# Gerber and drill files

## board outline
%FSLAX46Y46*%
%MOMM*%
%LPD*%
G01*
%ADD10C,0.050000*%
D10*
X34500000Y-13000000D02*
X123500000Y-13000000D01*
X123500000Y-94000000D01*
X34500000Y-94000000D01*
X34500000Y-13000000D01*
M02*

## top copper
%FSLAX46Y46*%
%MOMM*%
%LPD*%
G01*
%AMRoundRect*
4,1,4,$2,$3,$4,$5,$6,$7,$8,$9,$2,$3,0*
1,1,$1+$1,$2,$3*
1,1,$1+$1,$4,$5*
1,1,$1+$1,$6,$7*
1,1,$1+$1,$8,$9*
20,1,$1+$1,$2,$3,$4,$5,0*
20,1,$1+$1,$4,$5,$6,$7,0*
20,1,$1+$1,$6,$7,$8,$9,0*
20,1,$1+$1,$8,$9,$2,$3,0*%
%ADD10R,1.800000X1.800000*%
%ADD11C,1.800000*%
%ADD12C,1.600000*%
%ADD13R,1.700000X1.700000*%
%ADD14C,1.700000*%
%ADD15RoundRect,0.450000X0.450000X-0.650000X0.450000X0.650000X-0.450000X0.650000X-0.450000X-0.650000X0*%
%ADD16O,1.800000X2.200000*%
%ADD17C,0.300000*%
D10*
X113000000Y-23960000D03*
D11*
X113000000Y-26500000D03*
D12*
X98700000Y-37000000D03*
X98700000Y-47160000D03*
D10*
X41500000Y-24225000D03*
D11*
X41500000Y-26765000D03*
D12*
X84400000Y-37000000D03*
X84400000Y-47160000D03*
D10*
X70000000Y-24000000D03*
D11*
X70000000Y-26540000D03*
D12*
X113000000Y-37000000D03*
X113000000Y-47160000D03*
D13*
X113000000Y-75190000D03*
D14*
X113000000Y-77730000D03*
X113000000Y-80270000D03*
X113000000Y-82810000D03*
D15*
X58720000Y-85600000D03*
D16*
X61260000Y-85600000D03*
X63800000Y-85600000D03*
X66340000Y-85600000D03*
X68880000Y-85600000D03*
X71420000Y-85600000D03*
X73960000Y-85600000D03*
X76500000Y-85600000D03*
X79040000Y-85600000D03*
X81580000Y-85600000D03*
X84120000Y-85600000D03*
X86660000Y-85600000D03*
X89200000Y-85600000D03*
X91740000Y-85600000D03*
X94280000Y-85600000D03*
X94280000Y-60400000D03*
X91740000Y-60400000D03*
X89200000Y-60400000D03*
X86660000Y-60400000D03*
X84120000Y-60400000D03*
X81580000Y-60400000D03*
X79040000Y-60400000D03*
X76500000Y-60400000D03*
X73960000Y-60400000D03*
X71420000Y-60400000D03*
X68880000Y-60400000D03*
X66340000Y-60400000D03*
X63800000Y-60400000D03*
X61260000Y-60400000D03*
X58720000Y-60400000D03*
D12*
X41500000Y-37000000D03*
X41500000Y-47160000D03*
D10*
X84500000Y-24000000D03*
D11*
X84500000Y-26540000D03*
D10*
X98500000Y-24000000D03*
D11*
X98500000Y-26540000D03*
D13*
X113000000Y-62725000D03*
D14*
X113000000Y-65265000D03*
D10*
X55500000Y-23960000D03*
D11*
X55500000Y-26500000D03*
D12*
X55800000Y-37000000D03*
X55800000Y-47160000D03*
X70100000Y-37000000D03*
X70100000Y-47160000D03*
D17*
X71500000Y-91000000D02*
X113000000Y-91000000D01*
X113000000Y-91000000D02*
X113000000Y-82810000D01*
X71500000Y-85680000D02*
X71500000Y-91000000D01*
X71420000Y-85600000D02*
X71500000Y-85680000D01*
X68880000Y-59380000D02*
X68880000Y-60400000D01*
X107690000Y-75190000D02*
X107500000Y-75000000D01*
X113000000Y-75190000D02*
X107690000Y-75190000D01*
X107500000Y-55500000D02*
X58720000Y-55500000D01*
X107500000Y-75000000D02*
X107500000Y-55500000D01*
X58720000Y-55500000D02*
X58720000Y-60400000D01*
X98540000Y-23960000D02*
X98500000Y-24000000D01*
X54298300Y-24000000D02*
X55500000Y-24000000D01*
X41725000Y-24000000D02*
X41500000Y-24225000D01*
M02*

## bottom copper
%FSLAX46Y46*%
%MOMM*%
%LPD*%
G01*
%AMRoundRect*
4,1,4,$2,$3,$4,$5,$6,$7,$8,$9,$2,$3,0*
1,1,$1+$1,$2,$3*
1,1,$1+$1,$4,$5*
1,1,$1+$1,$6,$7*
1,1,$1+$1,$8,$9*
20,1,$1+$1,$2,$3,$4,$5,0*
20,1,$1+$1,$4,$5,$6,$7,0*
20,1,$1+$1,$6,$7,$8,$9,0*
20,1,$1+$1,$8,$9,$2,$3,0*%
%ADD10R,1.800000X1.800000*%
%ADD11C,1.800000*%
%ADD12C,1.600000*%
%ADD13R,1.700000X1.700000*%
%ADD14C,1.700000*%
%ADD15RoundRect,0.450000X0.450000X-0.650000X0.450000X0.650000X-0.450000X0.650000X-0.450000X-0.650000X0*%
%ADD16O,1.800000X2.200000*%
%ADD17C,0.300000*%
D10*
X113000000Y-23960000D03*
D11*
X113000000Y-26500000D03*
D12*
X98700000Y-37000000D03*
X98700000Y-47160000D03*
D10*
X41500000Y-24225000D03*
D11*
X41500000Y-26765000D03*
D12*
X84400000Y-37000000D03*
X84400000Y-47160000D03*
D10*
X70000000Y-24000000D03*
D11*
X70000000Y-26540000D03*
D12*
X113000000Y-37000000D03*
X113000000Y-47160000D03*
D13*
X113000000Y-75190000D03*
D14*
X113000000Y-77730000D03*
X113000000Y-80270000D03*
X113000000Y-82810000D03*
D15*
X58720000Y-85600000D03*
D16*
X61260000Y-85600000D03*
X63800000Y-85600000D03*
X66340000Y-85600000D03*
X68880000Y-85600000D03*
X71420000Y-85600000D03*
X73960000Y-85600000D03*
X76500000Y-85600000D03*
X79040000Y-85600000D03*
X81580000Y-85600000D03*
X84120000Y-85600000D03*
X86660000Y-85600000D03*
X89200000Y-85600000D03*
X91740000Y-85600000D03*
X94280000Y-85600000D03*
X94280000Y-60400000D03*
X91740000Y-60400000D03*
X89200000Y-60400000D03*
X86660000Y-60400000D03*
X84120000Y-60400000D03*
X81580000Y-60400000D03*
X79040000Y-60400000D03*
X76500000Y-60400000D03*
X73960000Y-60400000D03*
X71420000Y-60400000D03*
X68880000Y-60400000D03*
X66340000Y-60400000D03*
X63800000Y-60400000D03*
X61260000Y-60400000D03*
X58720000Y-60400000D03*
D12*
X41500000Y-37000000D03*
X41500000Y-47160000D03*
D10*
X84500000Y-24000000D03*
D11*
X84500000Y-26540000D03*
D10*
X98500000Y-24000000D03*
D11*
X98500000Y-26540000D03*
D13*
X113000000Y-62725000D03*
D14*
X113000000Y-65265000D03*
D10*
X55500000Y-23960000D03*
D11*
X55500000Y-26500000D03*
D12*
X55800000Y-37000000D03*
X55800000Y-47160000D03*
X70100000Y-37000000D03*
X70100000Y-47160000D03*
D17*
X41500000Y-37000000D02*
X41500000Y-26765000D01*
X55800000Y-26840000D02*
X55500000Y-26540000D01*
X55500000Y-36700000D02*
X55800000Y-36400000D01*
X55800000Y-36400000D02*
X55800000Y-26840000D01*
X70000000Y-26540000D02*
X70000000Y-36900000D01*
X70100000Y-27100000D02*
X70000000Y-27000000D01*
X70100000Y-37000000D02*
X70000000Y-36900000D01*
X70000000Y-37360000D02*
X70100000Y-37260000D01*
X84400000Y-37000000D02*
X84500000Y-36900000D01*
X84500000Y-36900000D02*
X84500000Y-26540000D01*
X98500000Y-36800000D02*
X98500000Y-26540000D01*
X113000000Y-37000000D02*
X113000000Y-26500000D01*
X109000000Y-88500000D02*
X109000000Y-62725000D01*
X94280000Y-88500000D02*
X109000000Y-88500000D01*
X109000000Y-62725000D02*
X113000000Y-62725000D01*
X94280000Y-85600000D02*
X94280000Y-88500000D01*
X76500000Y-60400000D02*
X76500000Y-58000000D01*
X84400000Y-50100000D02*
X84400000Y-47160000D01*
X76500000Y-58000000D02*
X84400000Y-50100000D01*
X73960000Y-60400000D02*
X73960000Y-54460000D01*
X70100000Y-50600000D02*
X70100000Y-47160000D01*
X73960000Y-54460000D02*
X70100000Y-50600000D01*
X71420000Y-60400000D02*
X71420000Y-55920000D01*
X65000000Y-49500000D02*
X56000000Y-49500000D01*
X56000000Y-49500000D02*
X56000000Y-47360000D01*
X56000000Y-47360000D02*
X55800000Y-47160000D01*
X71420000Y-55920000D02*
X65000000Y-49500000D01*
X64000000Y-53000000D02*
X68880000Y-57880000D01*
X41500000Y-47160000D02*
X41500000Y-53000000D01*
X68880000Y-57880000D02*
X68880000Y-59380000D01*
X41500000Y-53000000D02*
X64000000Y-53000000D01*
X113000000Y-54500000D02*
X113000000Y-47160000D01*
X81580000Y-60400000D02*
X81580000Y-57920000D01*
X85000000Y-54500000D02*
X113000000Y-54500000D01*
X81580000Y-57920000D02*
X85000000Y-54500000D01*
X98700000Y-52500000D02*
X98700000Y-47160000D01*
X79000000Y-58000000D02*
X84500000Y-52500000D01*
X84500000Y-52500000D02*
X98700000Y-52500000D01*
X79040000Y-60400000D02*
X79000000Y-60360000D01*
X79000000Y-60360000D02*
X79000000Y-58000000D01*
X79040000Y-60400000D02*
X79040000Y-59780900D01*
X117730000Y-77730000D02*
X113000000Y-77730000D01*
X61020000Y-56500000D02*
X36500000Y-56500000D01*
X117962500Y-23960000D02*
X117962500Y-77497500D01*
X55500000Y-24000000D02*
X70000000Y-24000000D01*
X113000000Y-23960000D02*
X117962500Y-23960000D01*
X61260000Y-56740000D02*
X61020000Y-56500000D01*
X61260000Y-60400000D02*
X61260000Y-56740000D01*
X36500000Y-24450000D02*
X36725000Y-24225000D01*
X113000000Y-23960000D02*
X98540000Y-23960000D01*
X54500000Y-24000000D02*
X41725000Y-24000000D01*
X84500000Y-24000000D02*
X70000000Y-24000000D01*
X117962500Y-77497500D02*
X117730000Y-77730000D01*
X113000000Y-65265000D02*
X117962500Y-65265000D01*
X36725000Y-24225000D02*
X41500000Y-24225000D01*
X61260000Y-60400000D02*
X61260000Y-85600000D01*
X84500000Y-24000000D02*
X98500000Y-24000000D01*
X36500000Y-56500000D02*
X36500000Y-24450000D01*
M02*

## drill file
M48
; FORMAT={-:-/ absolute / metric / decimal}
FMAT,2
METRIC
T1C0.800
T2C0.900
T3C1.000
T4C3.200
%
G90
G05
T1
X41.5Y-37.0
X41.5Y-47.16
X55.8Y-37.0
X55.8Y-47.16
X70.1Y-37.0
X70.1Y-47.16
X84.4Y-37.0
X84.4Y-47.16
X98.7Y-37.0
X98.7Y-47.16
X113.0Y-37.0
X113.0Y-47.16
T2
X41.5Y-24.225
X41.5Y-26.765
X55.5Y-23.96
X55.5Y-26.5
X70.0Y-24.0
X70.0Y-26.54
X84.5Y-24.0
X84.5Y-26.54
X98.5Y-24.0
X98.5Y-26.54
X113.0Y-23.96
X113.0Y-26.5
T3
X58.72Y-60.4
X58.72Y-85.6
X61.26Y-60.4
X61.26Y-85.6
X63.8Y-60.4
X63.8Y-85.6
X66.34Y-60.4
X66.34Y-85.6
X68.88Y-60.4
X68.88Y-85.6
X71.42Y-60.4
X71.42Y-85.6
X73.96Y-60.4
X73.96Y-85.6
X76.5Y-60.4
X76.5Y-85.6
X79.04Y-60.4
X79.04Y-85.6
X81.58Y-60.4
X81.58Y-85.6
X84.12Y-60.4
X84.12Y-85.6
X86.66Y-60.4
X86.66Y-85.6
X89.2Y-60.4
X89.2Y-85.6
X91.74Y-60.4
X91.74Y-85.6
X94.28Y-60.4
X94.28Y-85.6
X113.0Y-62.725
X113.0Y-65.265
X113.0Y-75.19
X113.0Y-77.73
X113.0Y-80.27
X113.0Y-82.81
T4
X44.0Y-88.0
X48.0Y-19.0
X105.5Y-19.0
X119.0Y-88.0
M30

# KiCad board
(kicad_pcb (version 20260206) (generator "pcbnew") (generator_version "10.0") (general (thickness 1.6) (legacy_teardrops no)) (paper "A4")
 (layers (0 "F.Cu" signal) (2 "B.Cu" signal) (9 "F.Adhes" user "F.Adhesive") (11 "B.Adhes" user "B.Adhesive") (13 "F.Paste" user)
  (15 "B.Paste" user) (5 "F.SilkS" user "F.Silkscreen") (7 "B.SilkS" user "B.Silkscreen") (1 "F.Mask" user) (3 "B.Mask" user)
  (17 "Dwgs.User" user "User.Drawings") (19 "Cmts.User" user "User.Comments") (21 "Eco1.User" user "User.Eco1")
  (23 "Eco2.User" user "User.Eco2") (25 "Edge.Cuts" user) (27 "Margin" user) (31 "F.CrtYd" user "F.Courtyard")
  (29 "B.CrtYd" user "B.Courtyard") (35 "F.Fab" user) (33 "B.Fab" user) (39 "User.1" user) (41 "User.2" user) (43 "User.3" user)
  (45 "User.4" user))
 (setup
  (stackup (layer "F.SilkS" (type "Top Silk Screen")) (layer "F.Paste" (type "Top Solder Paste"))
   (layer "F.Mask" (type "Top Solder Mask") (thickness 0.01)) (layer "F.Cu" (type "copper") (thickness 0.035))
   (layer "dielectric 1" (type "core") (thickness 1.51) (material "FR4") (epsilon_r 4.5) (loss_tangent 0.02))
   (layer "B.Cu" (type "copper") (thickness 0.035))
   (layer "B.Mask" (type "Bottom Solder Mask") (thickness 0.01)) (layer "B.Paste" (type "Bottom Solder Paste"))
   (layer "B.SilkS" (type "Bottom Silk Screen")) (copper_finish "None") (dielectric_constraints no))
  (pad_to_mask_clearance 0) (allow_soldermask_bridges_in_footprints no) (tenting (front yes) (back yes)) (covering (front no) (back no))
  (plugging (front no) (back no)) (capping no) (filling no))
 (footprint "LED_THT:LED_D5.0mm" (layer "F.Cu") (at 113 23.96 -90)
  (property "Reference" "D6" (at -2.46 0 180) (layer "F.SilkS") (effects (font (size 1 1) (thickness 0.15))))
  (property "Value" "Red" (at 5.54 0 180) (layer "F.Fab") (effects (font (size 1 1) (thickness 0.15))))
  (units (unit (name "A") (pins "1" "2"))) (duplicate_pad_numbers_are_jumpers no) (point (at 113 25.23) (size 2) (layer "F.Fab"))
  (pad "1" thru_hole rect (at 0 0 270) (size 1.8 1.8) (drill 0.9) (layers "*.Cu" "*.Mask") (remove_unused_layers no) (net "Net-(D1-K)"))
  (pad "2" thru_hole circle (at 2.54 0 270) (size 1.8 1.8) (drill 0.9) (layers "*.Cu" "*.Mask") (remove_unused_layers no) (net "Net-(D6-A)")))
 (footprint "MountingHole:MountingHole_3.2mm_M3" (layer "F.Cu") (at 44 88)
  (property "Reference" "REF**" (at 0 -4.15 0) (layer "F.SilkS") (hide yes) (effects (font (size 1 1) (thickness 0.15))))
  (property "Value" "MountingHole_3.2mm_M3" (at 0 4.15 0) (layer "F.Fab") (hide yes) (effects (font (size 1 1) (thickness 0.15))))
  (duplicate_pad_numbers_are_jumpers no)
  (pad "" np_thru_hole circle (at 0 0) (size 3.2 3.2) (drill 3.2) (layers "*.Cu" "*.Mask")))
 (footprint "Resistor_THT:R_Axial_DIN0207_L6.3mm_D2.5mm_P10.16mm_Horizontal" (layer "F.Cu") (at 98.7 37 -90)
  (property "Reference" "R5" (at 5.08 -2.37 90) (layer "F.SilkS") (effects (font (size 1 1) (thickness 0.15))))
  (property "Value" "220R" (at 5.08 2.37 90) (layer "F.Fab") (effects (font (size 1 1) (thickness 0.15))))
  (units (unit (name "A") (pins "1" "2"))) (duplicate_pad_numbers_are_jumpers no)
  (pad "1" thru_hole circle (at 0 0 270) (size 1.6 1.6) (drill 0.8) (layers "*.Cu" "*.Mask") (remove_unused_layers no) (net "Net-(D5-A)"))
  (pad "2" thru_hole circle (at 10.16 0 270) (size 1.6 1.6) (drill 0.8) (layers "*.Cu" "*.Mask") (remove_unused_layers no)
   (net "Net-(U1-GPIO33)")))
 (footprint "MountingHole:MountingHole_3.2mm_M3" (layer "F.Cu") (at 105.5 19)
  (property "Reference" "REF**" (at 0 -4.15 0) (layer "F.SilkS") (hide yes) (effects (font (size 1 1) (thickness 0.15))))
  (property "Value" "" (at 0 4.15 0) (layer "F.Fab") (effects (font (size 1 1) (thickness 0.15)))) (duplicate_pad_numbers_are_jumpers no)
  (pad "" np_thru_hole circle (at 0 0) (size 3.2 3.2) (drill 3.2) (layers "*.Cu" "*.Mask")))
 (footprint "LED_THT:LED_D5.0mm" (layer "F.Cu") (at 41.5 24.225 -90)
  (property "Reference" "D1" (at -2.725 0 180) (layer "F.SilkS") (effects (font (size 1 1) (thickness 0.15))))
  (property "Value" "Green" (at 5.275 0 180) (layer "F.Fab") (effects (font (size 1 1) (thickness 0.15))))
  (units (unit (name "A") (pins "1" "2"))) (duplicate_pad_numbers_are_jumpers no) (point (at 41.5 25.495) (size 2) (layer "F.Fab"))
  (pad "1" thru_hole rect (at 0 0 270) (size 1.8 1.8) (drill 0.9) (layers "*.Cu" "*.Mask") (remove_unused_layers no) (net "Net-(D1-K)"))
  (pad "2" thru_hole circle (at 2.54 0 270) (size 1.8 1.8) (drill 0.9) (layers "*.Cu" "*.Mask") (remove_unused_layers no) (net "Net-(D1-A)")))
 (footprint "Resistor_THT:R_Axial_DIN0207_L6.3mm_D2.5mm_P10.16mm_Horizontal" (layer "F.Cu") (at 84.4 37 -90)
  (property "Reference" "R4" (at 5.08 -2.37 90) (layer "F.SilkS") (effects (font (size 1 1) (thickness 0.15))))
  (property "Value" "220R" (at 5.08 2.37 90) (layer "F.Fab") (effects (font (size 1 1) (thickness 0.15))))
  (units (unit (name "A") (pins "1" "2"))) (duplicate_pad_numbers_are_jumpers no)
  (pad "1" thru_hole circle (at 0 0 270) (size 1.6 1.6) (drill 0.8) (layers "*.Cu" "*.Mask") (remove_unused_layers no) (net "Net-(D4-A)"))
  (pad "2" thru_hole circle (at 10.16 0 270) (size 1.6 1.6) (drill 0.8) (layers "*.Cu" "*.Mask") (remove_unused_layers no)
   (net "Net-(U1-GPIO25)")))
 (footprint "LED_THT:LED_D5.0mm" (layer "F.Cu") (at 70 24 -90)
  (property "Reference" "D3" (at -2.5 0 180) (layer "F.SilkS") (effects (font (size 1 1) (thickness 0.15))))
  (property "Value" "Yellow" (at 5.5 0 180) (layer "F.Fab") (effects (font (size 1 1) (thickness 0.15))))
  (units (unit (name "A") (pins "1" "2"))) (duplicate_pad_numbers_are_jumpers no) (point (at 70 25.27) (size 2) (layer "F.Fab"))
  (pad "1" thru_hole rect (at 0 0 270) (size 1.8 1.8) (drill 0.9) (layers "*.Cu" "*.Mask") (remove_unused_layers no) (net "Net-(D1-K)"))
  (pad "2" thru_hole circle (at 2.54 0 270) (size 1.8 1.8) (drill 0.9) (layers "*.Cu" "*.Mask") (remove_unused_layers no) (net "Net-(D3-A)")))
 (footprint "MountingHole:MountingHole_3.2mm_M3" (layer "F.Cu") (at 119 88)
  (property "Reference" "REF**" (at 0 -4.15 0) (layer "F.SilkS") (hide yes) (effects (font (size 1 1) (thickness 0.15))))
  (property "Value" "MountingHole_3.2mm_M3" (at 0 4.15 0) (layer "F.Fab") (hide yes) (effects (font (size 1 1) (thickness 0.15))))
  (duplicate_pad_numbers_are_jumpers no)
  (pad "" np_thru_hole circle (at 0 0) (size 3.2 3.2) (drill 3.2) (layers "*.Cu" "*.Mask")))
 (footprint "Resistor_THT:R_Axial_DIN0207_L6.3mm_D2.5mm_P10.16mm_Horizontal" (layer "F.Cu") (at 113 37 -90)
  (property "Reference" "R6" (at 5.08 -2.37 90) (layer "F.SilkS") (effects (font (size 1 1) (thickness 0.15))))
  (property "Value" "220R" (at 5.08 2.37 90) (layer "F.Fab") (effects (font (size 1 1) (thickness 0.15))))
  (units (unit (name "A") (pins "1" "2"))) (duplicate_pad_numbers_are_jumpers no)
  (pad "1" thru_hole circle (at 0 0 270) (size 1.6 1.6) (drill 0.8) (layers "*.Cu" "*.Mask") (remove_unused_layers no) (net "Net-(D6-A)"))
  (pad "2" thru_hole circle (at 10.16 0 270) (size 1.6 1.6) (drill 0.8) (layers "*.Cu" "*.Mask") (remove_unused_layers no)
   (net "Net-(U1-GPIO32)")))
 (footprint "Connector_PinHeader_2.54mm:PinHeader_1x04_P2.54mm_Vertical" (layer "F.Cu") (at 113 75.19)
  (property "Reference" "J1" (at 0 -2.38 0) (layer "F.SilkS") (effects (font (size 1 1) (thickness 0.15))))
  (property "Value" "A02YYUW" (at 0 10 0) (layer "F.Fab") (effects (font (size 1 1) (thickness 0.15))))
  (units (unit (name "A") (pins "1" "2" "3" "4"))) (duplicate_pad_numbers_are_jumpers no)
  (pad "1" thru_hole rect (at 0 0) (size 1.7 1.7) (drill 1) (layers "*.Cu" "*.Mask") (remove_unused_layers no) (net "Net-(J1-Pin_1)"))
  (pad "2" thru_hole circle (at 0 2.54) (size 1.7 1.7) (drill 1) (layers "*.Cu" "*.Mask") (remove_unused_layers no) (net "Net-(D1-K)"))
  (pad "3" thru_hole circle (at 0 5.08) (size 1.7 1.7) (drill 1) (layers "*.Cu" "*.Mask") (remove_unused_layers no)
   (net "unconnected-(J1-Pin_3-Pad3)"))
  (pad "4" thru_hole circle (at 0 7.62) (size 1.7 1.7) (drill 1) (layers "*.Cu" "*.Mask") (remove_unused_layers no) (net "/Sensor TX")))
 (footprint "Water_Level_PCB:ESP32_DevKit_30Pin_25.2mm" (layer "F.Cu") (at 76.5 73 90)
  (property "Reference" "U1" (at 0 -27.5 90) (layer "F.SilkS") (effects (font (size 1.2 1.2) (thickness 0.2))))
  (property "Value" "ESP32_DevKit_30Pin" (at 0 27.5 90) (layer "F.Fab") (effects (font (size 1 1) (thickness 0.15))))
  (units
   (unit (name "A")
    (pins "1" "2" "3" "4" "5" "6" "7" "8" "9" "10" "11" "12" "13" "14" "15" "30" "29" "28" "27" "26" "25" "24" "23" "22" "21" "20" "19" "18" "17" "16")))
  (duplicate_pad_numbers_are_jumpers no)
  (pad "1" thru_hole roundrect (at -12.6 -17.78 90) (size 2.2 1.8) (drill 1) (layers "*.Cu" "*.Mask") (remove_unused_layers no)
   (roundrect_rratio 0.25) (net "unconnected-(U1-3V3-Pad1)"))
  (pad "2" thru_hole oval (at -12.6 -15.24 90) (size 2.2 1.8) (drill 1) (layers "*.Cu" "*.Mask") (remove_unused_layers no)
   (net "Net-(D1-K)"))
  (pad "3" thru_hole oval (at -12.6 -12.7 90) (size 2.2 1.8) (drill 1) (layers "*.Cu" "*.Mask") (remove_unused_layers no)
   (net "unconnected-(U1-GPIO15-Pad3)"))
  (pad "4" thru_hole oval (at -12.6 -10.16 90) (size 2.2 1.8) (drill 1) (layers "*.Cu" "*.Mask") (remove_unused_layers no)
   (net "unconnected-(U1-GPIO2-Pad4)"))
  (pad "5" thru_hole oval (at -12.6 -7.62 90) (size 2.2 1.8) (drill 1) (layers "*.Cu" "*.Mask") (remove_unused_layers no)
   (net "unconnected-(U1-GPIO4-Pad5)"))
  (pad "6" thru_hole oval (at -12.6 -5.08 90) (size 2.2 1.8) (drill 1) (layers "*.Cu" "*.Mask") (remove_unused_layers no) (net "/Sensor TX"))
  (pad "7" thru_hole oval (at -12.6 -2.54 90) (size 2.2 1.8) (drill 1) (layers "*.Cu" "*.Mask") (remove_unused_layers no)
   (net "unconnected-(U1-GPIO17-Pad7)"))
  (pad "8" thru_hole oval (at -12.6 0 90) (size 2.2 1.8) (drill 1) (layers "*.Cu" "*.Mask") (remove_unused_layers no)
   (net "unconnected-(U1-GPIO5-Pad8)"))
  (pad "9" thru_hole oval (at -12.6 2.54 90) (size 2.2 1.8) (drill 1) (layers "*.Cu" "*.Mask") (remove_unused_layers no)
   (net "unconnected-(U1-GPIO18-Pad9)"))
  (pad "10" thru_hole oval (at -12.6 5.08 90) (size 2.2 1.8) (drill 1) (layers "*.Cu" "*.Mask") (remove_unused_layers no)
   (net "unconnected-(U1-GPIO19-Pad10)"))
  (pad "11" thru_hole oval (at -12.6 7.62 90) (size 2.2 1.8) (drill 1) (layers "*.Cu" "*.Mask") (remove_unused_layers no)
   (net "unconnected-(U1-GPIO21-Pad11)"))
  (pad "12" thru_hole oval (at -12.6 10.16 90) (size 2.2 1.8) (drill 1) (layers "*.Cu" "*.Mask") (remove_unused_layers no)
   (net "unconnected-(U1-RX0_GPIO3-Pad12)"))
  (pad "13" thru_hole oval (at -12.6 12.7 90) (size 2.2 1.8) (drill 1) (layers "*.Cu" "*.Mask") (remove_unused_layers no)
   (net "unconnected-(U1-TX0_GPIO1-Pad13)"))
  (pad "14" thru_hole oval (at -12.6 15.24 90) (size 2.2 1.8) (drill 1) (layers "*.Cu" "*.Mask") (remove_unused_layers no)
   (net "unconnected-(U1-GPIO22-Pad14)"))
  (pad "15" thru_hole oval (at -12.6 17.78 90) (size 2.2 1.8) (drill 1) (layers "*.Cu" "*.Mask") (remove_unused_layers no)
   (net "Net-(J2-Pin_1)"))
  (pad "16" thru_hole oval (at 12.6 17.78 90) (size 2.2 1.8) (drill 1) (layers "*.Cu" "*.Mask") (remove_unused_layers no)
   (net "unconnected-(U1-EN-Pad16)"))
  (pad "17" thru_hole oval (at 12.6 15.24 90) (size 2.2 1.8) (drill 1) (layers "*.Cu" "*.Mask") (remove_unused_layers no)
   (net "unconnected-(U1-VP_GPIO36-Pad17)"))
  (pad "18" thru_hole oval (at 12.6 12.7 90) (size 2.2 1.8) (drill 1) (layers "*.Cu" "*.Mask") (remove_unused_layers no)
   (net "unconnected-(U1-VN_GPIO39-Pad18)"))
  (pad "19" thru_hole oval (at 12.6 10.16 90) (size 2.2 1.8) (drill 1) (layers "*.Cu" "*.Mask") (remove_unused_layers no)
   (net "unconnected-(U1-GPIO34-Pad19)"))
  (pad "20" thru_hole oval (at 12.6 7.62 90) (size 2.2 1.8) (drill 1) (layers "*.Cu" "*.Mask") (remove_unused_layers no)
   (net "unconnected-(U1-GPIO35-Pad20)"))
  (pad "21" thru_hole oval (at 12.6 5.08 90) (size 2.2 1.8) (drill 1) (layers "*.Cu" "*.Mask") (remove_unused_layers no)
   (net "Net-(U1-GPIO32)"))
  (pad "22" thru_hole oval (at 12.6 2.54 90) (size 2.2 1.8) (drill 1) (layers "*.Cu" "*.Mask") (remove_unused_layers no)
   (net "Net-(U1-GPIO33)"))
  (pad "23" thru_hole oval (at 12.6 0 90) (size 2.2 1.8) (drill 1) (layers "*.Cu" "*.Mask") (remove_unused_layers no)
   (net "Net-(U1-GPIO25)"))
  (pad "24" thru_hole oval (at 12.6 -2.54 90) (size 2.2 1.8) (drill 1) (layers "*.Cu" "*.Mask") (remove_unused_layers no)
   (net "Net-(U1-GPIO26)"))
  (pad "25" thru_hole oval (at 12.6 -5.08 90) (size 2.2 1.8) (drill 1) (layers "*.Cu" "*.Mask") (remove_unused_layers no)
   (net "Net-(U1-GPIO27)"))
  (pad "26" thru_hole oval (at 12.6 -7.62 90) (size 2.2 1.8) (drill 1) (layers "*.Cu" "*.Mask") (remove_unused_layers no)
   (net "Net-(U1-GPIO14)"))
  (pad "27" thru_hole oval (at 12.6 -10.16 90) (size 2.2 1.8) (drill 1) (layers "*.Cu" "*.Mask") (remove_unused_layers no)
   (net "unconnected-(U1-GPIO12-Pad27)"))
  (pad "28" thru_hole oval (at 12.6 -12.7 90) (size 2.2 1.8) (drill 1) (layers "*.Cu" "*.Mask") (remove_unused_layers no)
   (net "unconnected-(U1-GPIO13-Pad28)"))
  (pad "29" thru_hole oval (at 12.6 -15.24 90) (size 2.2 1.8) (drill 1) (layers "*.Cu" "*.Mask") (remove_unused_layers no)
   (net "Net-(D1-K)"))
  (pad "30" thru_hole oval (at 12.6 -17.78 90) (size 2.2 1.8) (drill 1) (layers "*.Cu" "*.Mask") (remove_unused_layers no)
   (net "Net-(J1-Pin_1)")))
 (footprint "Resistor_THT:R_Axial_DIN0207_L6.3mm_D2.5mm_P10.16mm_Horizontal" (layer "F.Cu") (at 41.5 37 -90)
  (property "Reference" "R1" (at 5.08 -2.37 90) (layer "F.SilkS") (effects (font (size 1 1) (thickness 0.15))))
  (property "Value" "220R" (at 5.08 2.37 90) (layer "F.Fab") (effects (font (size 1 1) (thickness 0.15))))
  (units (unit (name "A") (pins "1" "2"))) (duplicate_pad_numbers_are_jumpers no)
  (pad "1" thru_hole circle (at 0 0 270) (size 1.6 1.6) (drill 0.8) (layers "*.Cu" "*.Mask") (remove_unused_layers no) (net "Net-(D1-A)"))
  (pad "2" thru_hole circle (at 10.16 0 270) (size 1.6 1.6) (drill 0.8) (layers "*.Cu" "*.Mask") (remove_unused_layers no)
   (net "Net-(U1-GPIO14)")))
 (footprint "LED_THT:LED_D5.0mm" (layer "F.Cu") (at 84.5 24 -90)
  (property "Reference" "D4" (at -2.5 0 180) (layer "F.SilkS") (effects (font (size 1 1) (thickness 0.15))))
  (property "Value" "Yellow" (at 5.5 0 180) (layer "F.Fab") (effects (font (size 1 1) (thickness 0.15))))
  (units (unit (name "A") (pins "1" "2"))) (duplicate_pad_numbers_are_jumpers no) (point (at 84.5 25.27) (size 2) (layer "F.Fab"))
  (pad "1" thru_hole rect (at 0 0 270) (size 1.8 1.8) (drill 0.9) (layers "*.Cu" "*.Mask") (remove_unused_layers no) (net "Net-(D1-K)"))
  (pad "2" thru_hole circle (at 2.54 0 270) (size 1.8 1.8) (drill 0.9) (layers "*.Cu" "*.Mask") (remove_unused_layers no) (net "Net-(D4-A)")))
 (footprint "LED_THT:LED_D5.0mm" (layer "F.Cu") (at 98.5 24 -90)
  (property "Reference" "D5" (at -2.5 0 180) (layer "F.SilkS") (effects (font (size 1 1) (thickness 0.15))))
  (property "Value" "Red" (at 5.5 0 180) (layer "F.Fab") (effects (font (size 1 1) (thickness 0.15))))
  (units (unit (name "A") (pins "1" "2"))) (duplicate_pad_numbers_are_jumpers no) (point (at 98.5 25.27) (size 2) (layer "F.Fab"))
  (pad "1" thru_hole rect (at 0 0 270) (size 1.8 1.8) (drill 0.9) (layers "*.Cu" "*.Mask") (remove_unused_layers no) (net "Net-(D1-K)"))
  (pad "2" thru_hole circle (at 2.54 0 270) (size 1.8 1.8) (drill 0.9) (layers "*.Cu" "*.Mask") (remove_unused_layers no) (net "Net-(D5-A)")))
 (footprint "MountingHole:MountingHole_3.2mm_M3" (layer "F.Cu") (at 48 19)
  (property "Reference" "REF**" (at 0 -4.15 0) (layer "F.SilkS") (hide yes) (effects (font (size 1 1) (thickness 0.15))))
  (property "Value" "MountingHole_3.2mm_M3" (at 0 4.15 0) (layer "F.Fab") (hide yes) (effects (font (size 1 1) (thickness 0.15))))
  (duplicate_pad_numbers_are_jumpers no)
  (pad "" np_thru_hole circle (at 0 0) (size 3.2 3.2) (drill 3.2) (layers "*.Cu" "*.Mask")))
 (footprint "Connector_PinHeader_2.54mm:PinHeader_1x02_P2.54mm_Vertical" (layer "F.Cu") (at 113 62.725)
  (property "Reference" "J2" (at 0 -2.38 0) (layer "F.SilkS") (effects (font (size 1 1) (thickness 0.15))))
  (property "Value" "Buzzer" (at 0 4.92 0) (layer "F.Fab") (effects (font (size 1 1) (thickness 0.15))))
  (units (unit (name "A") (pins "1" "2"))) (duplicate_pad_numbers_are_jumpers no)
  (pad "1" thru_hole rect (at 0 0) (size 1.7 1.7) (drill 1) (layers "*.Cu" "*.Mask") (remove_unused_layers no) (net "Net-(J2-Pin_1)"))
  (pad "2" thru_hole circle (at 0 2.54) (size 1.7 1.7) (drill 1) (layers "*.Cu" "*.Mask") (remove_unused_layers no) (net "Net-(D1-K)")))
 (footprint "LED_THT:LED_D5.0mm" (layer "F.Cu") (at 55.5 23.96 -90)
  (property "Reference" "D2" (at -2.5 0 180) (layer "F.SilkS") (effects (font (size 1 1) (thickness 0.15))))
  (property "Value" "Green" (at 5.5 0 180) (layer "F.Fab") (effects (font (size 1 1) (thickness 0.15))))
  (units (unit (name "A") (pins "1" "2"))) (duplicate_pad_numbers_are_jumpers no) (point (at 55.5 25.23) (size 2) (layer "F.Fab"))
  (pad "1" thru_hole rect (at 0 0 270) (size 1.8 1.8) (drill 0.9) (layers "*.Cu" "*.Mask") (remove_unused_layers no) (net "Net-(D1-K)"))
  (pad "2" thru_hole circle (at 2.54 0 270) (size 1.8 1.8) (drill 0.9) (layers "*.Cu" "*.Mask") (remove_unused_layers no) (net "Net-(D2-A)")))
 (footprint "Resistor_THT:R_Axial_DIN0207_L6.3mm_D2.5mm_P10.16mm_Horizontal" (layer "F.Cu") (at 55.8 37 -90)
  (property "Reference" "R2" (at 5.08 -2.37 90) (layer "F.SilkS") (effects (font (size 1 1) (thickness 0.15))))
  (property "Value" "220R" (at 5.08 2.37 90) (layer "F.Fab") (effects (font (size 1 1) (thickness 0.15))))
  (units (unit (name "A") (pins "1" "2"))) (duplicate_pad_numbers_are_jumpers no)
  (pad "1" thru_hole circle (at 0 0 270) (size 1.6 1.6) (drill 0.8) (layers "*.Cu" "*.Mask") (remove_unused_layers no) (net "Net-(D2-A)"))
  (pad "2" thru_hole circle (at 10.16 0 270) (size 1.6 1.6) (drill 0.8) (layers "*.Cu" "*.Mask") (remove_unused_layers no)
   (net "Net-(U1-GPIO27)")))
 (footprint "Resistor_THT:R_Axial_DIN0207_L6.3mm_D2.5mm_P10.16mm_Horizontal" (layer "F.Cu") (at 70.1 37 -90)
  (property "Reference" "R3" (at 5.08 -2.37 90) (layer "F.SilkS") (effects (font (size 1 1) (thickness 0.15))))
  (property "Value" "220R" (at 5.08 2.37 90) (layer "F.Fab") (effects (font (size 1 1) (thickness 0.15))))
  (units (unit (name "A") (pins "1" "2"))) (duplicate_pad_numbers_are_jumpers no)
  (pad "1" thru_hole circle (at 0 0 270) (size 1.6 1.6) (drill 0.8) (layers "*.Cu" "*.Mask") (remove_unused_layers no) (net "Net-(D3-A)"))
  (pad "2" thru_hole circle (at 10.16 0 270) (size 1.6 1.6) (drill 0.8) (layers "*.Cu" "*.Mask") (remove_unused_layers no)
   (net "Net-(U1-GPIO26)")))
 (gr_rect (start 34.5 13) (end 123.5 94) (stroke (width 0.05) (type default)) (fill no) (layer "Edge.Cuts"))
 (segment (start 41.5 37) (end 41.5 26.765) (width 0.3) (layer "B.Cu") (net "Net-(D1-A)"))
 (segment (start 55.8 26.84) (end 55.5 26.54) (width 0.3) (layer "B.Cu") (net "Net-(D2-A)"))
 (segment (start 55.5 36.7) (end 55.8 36.4) (width 0.3) (layer "B.Cu") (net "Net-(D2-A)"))
 (segment (start 55.8 36.4) (end 55.8 26.84) (width 0.3) (layer "B.Cu") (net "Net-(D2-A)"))
 (segment (start 70 26.54) (end 70 36.9) (width 0.3) (layer "B.Cu") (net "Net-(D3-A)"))
 (segment (start 70.1 27.1) (end 70 27) (width 0.3) (layer "B.Cu") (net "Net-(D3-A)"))
 (segment (start 70.1 37) (end 70 36.9) (width 0.3) (layer "B.Cu") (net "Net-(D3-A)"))
 (segment (start 70 37.36) (end 70.1 37.26) (width 0.3) (layer "B.Cu") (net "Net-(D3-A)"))
 (segment (start 84.4 37) (end 84.5 36.9) (width 0.3) (layer "B.Cu") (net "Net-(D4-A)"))
 (segment (start 84.5 36.9) (end 84.5 26.54) (width 0.3) (layer "B.Cu") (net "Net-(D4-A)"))
 (segment (start 98.5 36.8) (end 98.5 26.54) (width 0.3) (layer "B.Cu") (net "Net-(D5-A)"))
 (segment (start 113 37) (end 113 26.5) (width 0.3) (layer "B.Cu") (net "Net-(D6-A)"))
 (segment (start 71.5 91) (end 113 91) (width 0.3) (layer "F.Cu") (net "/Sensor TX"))
 (segment (start 113 91) (end 113 82.81) (width 0.3) (layer "F.Cu") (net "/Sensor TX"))
 (segment (start 71.5 85.68) (end 71.5 91) (width 0.3) (layer "F.Cu") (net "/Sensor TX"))
 (segment (start 71.42 85.6) (end 71.5 85.68) (width 0.3) (layer "F.Cu") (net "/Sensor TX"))
 (segment (start 109 88.5) (end 109 62.725) (width 0.3) (layer "B.Cu") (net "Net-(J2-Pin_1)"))
 (segment (start 94.28 88.5) (end 109 88.5) (width 0.3) (layer "B.Cu") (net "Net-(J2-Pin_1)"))
 (segment (start 109 62.725) (end 113 62.725) (width 0.3) (layer "B.Cu") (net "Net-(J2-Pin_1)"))
 (segment (start 94.28 85.6) (end 94.28 88.5) (width 0.3) (layer "B.Cu") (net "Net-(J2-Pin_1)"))
 (segment (start 76.5 60.4) (end 76.5 58) (width 0.3) (layer "B.Cu") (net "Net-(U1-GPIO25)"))
 (segment (start 84.4 50.1) (end 84.4 47.16) (width 0.3) (layer "B.Cu") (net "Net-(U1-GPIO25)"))
 (segment (start 76.5 58) (end 84.4 50.1) (width 0.3) (layer "B.Cu") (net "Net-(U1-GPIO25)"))
 (segment (start 73.96 60.4) (end 73.96 54.46) (width 0.3) (layer "B.Cu") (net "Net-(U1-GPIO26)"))
 (segment (start 70.1 50.6) (end 70.1 47.16) (width 0.3) (layer "B.Cu") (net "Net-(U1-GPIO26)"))
 (segment (start 73.96 54.46) (end 70.1 50.6) (width 0.3) (layer "B.Cu") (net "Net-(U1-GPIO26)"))
 (segment (start 71.42 60.4) (end 71.42 55.92) (width 0.3) (layer "B.Cu") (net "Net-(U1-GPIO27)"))
 (segment (start 65 49.5) (end 56 49.5) (width 0.3) (layer "B.Cu") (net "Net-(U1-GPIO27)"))
 (segment (start 56 49.5) (end 56 47.36) (width 0.3) (layer "B.Cu") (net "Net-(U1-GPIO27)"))
 (segment (start 56 47.36) (end 55.8 47.16) (width 0.3) (layer "B.Cu") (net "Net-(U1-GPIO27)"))
 (segment (start 71.42 55.92) (end 65 49.5) (width 0.3) (layer "B.Cu") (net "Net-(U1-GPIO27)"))
 (segment (start 68.88 59.38) (end 68.88 60.4) (width 0.3) (layer "F.Cu") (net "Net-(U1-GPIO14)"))
 (segment (start 64 53) (end 68.88 57.88) (width 0.3) (layer "B.Cu") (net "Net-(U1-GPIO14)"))
 (segment (start 41.5 47.16) (end 41.5 53) (width 0.3) (layer "B.Cu") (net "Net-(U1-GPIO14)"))
 (segment (start 68.88 57.88) (end 68.88 59.38) (width 0.3) (layer "B.Cu") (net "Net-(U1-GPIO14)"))
 (segment (start 41.5 53) (end 64 53) (width 0.3) (layer "B.Cu") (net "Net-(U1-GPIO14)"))
 (segment (start 113 54.5) (end 113 47.16) (width 0.3) (layer "B.Cu") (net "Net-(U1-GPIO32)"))
 (segment (start 81.58 60.4) (end 81.58 57.92) (width 0.3) (layer "B.Cu") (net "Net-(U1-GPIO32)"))
 (segment (start 85 54.5) (end 113 54.5) (width 0.3) (layer "B.Cu") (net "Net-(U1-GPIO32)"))
 (segment (start 81.58 57.92) (end 85 54.5) (width 0.3) (layer "B.Cu") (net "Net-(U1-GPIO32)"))
 (segment (start 98.7 52.5) (end 98.7 47.16) (width 0.3) (layer "B.Cu") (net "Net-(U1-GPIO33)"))
 (segment (start 79 58) (end 84.5 52.5) (width 0.3) (layer "B.Cu") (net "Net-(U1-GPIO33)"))
 (segment (start 84.5 52.5) (end 98.7 52.5) (width 0.3) (layer "B.Cu") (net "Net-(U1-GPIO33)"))
 (segment (start 79.04 60.4) (end 79 60.36) (width 0.3) (layer "B.Cu") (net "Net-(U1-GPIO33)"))
 (segment (start 79 60.36) (end 79 58) (width 0.3) (layer "B.Cu") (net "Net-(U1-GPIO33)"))
 (segment (start 79.04 60.4) (end 79.04 59.7809) (width 0.3) (layer "B.Cu") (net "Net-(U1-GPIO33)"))
 (segment (start 107.69 75.19) (end 107.5 75) (width 0.3) (layer "F.Cu") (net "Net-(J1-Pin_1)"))
 (segment (start 113 75.19) (end 107.69 75.19) (width 0.3) (layer "F.Cu") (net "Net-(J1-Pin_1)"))
 (segment (start 107.5 55.5) (end 58.72 55.5) (width 0.3) (layer "F.Cu") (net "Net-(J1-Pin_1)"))
 (segment (start 107.5 75) (end 107.5 55.5) (width 0.3) (layer "F.Cu") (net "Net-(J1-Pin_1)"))
 (segment (start 58.72 55.5) (end 58.72 60.4) (width 0.3) (layer "F.Cu") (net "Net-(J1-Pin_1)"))
 (segment (start 98.54 23.96) (end 98.5 24) (width 0.3) (layer "F.Cu") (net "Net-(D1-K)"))
 (segment (start 54.2983 24) (end 55.5 24) (width 0.3) (layer "F.Cu") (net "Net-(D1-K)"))
 (segment (start 41.725 24) (end 41.5 24.225) (width 0.3) (layer "F.Cu") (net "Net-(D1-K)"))
 (segment (start 117.73 77.73) (end 113 77.73) (width 0.3) (layer "B.Cu") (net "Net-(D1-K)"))
 (segment (start 61.02 56.5) (end 36.5 56.5) (width 0.3) (layer "B.Cu") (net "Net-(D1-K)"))
 (segment (start 117.9625 23.96) (end 117.9625 77.4975) (width 0.3) (layer "B.Cu") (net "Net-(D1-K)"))
 (segment (start 55.5 24) (end 70 24) (width 0.3) (layer "B.Cu") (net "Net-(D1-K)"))
 (segment (start 113 23.96) (end 117.9625 23.96) (width 0.3) (layer "B.Cu") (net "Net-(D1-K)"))
 (segment (start 61.26 56.74) (end 61.02 56.5) (width 0.3) (layer "B.Cu") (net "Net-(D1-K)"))
 (segment (start 61.26 60.4) (end 61.26 56.74) (width 0.3) (layer "B.Cu") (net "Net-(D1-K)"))
 (segment (start 36.5 24.45) (end 36.725 24.225) (width 0.3) (layer "B.Cu") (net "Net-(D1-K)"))
 (segment (start 113 23.96) (end 98.54 23.96) (width 0.3) (layer "B.Cu") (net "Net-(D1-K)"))
 (segment (start 54.5 24) (end 41.725 24) (width 0.3) (layer "B.Cu") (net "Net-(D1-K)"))
 (segment (start 84.5 24) (end 70 24) (width 0.3) (layer "B.Cu") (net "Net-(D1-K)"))
 (segment (start 117.9625 77.4975) (end 117.73 77.73) (width 0.3) (layer "B.Cu") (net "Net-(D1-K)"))
 (segment (start 113 65.265) (end 117.9625 65.265) (width 0.3) (layer "B.Cu") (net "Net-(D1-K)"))
 (segment (start 36.725 24.225) (end 41.5 24.225) (width 0.3) (layer "B.Cu") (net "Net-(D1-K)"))
 (segment (start 61.26 60.4) (end 61.26 85.6) (width 0.3) (layer "B.Cu") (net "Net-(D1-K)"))
 (segment (start 84.5 24) (end 98.5 24) (width 0.3) (layer "B.Cu") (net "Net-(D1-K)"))
 (segment (start 36.5 56.5) (end 36.5 24.45) (width 0.3) (layer "B.Cu") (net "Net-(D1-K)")))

